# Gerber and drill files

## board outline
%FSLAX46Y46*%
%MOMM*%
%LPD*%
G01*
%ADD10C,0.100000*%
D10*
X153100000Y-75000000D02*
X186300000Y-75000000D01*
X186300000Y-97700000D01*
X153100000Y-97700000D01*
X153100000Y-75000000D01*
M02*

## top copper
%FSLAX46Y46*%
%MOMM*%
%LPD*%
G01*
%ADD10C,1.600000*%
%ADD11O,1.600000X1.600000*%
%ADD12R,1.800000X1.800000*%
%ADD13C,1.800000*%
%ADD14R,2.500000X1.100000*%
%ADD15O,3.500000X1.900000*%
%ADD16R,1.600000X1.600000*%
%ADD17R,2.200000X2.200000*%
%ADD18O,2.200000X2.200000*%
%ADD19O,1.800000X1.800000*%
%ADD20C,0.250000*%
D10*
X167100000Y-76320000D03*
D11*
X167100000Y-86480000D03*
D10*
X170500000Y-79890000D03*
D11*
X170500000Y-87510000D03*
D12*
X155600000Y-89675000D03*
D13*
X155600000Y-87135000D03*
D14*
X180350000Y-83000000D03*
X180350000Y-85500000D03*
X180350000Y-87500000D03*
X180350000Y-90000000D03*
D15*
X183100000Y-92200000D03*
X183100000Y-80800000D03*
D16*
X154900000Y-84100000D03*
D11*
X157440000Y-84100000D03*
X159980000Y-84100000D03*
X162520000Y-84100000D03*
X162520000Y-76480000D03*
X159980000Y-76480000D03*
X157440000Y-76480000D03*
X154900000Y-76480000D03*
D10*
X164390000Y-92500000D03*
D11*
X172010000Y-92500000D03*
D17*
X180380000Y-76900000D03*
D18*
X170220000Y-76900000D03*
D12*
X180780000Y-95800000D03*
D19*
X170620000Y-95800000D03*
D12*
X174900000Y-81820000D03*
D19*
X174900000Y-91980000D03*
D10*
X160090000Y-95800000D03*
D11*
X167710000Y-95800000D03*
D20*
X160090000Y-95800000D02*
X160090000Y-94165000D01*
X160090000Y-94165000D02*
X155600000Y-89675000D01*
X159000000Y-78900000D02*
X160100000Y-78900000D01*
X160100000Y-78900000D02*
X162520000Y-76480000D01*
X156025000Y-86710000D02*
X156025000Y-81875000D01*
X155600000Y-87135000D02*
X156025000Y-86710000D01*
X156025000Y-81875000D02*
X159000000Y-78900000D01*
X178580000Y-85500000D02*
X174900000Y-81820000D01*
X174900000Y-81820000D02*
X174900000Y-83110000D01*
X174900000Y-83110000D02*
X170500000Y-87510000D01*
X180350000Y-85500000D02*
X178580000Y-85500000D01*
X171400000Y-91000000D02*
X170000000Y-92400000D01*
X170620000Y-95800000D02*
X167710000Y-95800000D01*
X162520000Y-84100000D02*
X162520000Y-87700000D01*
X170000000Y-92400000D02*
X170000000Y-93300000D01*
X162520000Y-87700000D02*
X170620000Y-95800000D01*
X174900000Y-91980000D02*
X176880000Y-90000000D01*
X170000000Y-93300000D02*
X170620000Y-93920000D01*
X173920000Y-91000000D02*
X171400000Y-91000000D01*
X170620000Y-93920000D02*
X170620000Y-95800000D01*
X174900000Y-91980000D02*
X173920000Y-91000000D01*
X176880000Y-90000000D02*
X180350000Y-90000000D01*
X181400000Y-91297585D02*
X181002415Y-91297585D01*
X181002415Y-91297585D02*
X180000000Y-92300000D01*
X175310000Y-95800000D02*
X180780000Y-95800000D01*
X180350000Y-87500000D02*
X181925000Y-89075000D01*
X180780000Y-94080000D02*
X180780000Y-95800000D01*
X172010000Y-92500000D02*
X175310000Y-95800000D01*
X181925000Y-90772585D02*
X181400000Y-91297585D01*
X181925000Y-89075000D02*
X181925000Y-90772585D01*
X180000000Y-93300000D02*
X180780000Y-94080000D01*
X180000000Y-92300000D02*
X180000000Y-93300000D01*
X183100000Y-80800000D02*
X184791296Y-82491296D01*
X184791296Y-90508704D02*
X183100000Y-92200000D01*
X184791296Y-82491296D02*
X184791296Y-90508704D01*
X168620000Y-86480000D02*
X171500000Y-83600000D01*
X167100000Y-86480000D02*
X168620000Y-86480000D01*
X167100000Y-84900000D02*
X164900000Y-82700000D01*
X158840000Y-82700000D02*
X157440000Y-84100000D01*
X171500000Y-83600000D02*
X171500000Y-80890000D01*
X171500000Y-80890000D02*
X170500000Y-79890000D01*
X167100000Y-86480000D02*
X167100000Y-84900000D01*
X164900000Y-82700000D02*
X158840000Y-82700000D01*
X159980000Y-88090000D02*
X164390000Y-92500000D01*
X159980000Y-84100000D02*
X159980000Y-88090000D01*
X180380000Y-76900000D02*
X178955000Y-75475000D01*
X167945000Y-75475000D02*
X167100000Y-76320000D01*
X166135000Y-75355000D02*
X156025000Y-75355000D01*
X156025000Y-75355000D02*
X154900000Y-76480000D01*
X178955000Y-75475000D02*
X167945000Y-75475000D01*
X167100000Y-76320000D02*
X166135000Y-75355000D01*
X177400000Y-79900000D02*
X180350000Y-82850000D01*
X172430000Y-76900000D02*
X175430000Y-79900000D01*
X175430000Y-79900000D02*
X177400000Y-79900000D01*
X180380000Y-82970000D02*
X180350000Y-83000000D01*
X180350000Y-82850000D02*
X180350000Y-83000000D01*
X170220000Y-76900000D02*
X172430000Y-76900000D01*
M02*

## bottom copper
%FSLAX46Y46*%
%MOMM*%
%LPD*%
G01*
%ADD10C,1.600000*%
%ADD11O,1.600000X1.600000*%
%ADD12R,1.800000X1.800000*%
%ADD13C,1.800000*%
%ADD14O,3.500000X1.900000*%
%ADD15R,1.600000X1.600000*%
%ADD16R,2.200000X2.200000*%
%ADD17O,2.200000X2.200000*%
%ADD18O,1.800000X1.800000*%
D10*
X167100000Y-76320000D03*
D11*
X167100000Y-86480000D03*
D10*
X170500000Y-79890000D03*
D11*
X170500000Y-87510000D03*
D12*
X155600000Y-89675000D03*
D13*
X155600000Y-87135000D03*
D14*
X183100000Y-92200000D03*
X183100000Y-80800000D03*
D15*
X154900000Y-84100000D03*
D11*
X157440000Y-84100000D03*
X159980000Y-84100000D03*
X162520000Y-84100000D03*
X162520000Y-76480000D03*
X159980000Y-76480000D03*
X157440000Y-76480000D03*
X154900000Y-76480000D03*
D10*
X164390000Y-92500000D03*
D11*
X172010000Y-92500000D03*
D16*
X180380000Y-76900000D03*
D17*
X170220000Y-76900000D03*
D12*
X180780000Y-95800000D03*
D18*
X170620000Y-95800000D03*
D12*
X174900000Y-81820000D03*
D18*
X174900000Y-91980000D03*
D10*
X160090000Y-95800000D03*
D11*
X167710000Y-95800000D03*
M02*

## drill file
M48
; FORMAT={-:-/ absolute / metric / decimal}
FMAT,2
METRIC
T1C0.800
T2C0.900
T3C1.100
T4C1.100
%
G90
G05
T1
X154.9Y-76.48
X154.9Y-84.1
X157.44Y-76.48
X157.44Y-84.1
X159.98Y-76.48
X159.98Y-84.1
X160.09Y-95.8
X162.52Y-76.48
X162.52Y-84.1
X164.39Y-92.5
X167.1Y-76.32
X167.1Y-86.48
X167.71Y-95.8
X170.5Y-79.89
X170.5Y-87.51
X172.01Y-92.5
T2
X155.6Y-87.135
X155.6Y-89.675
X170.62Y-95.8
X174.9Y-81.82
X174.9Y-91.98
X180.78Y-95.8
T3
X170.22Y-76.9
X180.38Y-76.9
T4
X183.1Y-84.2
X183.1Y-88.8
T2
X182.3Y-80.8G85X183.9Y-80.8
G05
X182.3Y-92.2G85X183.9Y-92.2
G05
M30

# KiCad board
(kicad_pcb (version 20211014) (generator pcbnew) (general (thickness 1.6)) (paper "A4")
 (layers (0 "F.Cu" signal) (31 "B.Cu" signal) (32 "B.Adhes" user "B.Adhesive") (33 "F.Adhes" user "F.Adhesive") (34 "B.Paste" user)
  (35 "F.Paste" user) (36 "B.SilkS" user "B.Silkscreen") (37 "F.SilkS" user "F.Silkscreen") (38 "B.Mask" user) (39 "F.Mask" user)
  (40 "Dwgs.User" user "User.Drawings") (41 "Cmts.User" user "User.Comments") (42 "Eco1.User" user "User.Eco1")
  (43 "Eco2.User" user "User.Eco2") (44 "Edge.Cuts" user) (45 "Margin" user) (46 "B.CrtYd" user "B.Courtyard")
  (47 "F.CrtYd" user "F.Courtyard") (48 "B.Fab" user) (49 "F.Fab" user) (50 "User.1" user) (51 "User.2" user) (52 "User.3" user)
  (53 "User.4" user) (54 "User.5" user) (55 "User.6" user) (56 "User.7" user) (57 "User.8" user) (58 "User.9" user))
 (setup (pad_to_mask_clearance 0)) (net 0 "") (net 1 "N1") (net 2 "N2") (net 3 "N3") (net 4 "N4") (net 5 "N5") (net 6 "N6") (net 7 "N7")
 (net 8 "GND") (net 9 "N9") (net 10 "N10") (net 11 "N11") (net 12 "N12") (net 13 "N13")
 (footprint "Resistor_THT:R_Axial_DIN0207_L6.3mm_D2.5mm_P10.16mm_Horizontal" (layer "F.Cu") (at 167.1 76.32 -90)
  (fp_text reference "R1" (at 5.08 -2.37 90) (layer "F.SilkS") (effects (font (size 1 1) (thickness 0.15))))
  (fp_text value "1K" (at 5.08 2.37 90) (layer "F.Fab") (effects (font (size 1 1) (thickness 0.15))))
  (pad "1" thru_hole circle (at 0 0 270) (size 1.6 1.6) (drill 0.8) (layers *.Cu *.Mask) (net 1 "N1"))
  (pad "2" thru_hole oval (at 10.16 0 270) (size 1.6 1.6) (drill 0.8) (layers *.Cu *.Mask) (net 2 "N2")))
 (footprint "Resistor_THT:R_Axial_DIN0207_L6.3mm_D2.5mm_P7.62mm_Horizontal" (layer "F.Cu") (at 170.5 79.89 -90)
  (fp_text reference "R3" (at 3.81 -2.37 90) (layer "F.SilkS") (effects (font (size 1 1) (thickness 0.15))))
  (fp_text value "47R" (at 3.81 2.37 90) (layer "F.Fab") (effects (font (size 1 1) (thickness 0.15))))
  (pad "1" thru_hole circle (at 0 0 270) (size 1.6 1.6) (drill 0.8) (layers *.Cu *.Mask) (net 2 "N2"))
  (pad "2" thru_hole oval (at 7.62 0 270) (size 1.6 1.6) (drill 0.8) (layers *.Cu *.Mask) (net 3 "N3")))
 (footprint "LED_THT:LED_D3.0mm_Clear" (layer "F.Cu") (at 155.6 89.675 90)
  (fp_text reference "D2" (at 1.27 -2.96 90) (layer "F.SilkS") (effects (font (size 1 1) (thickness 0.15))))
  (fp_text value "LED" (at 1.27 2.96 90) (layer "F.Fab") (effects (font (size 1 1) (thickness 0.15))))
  (pad "1" thru_hole rect (at 0 0 90) (size 1.8 1.8) (drill 0.9) (layers *.Cu *.Mask) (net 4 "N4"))
  (pad "2" thru_hole circle (at 2.54 0 90) (size 1.8 1.8) (drill 0.9) (layers *.Cu *.Mask) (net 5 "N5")))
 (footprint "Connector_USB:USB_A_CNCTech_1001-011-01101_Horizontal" (layer "F.Cu") (at 190 86.5)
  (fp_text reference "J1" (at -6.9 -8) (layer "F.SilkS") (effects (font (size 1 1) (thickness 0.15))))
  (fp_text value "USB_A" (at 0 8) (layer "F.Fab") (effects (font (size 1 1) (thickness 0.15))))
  (pad "" np_thru_hole circle (at -6.9 -2.3) (size 1.1 1.1) (drill 1.1) (layers *.Cu *.Mask))
  (pad "" np_thru_hole circle (at -6.9 2.3) (size 1.1 1.1) (drill 1.1) (layers *.Cu *.Mask))
  (pad "1" smd rect (at -9.65 -3.5) (size 2.5 1.1) (layers "F.Cu" "F.Paste" "F.Mask") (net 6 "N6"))
  (pad "2" smd rect (at -9.65 -1) (size 2.5 1.1) (layers "F.Cu" "F.Paste" "F.Mask") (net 3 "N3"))
  (pad "3" smd rect (at -9.65 1) (size 2.5 1.1) (layers "F.Cu" "F.Paste" "F.Mask") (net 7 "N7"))
  (pad "4" smd rect (at -9.65 3.5) (size 2.5 1.1) (layers "F.Cu" "F.Paste" "F.Mask") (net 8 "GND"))
  (pad "5" thru_hole oval (at -6.9 5.7) (size 3.5 1.9) (drill oval 2.5 0.9) (layers *.Cu *.Mask) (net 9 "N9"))
  (pad "5" thru_hole oval (at -6.9 -5.7) (size 3.5 1.9) (drill oval 2.5 0.9) (layers *.Cu *.Mask) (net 9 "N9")))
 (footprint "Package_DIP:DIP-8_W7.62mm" (layer "F.Cu") (at 154.9 84.1 90)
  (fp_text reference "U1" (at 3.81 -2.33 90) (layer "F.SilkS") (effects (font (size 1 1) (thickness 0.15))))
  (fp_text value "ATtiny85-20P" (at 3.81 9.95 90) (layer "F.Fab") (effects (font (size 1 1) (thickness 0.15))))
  (pad "1" thru_hole rect (at 0 0 90) (size 1.6 1.6) (drill 0.8) (layers *.Cu *.Mask) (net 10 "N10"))
  (pad "2" thru_hole oval (at 0 2.54 90) (size 1.6 1.6) (drill 0.8) (layers *.Cu *.Mask) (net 2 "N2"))
  (pad "3" thru_hole oval (at 0 5.08 90) (size 1.6 1.6) (drill 0.8) (layers *.Cu *.Mask) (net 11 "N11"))
  (pad "4" thru_hole oval (at 0 7.62 90) (size 1.6 1.6) (drill 0.8) (layers *.Cu *.Mask) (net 8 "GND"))
  (pad "5" thru_hole oval (at 7.62 7.62 90) (size 1.6 1.6) (drill 0.8) (layers *.Cu *.Mask) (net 5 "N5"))
  (pad "6" thru_hole oval (at 7.62 5.08 90) (size 1.6 1.6) (drill 0.8) (layers *.Cu *.Mask) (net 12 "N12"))
  (pad "7" thru_hole oval (at 7.62 2.54 90) (size 1.6 1.6) (drill 0.8) (layers *.Cu *.Mask) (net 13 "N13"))
  (pad "8" thru_hole oval (at 7.62 0 90) (size 1.6 1.6) (drill 0.8) (layers *.Cu *.Mask) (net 1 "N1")))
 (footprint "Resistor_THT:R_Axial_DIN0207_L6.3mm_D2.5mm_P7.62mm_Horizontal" (layer "F.Cu") (at 164.39 92.5)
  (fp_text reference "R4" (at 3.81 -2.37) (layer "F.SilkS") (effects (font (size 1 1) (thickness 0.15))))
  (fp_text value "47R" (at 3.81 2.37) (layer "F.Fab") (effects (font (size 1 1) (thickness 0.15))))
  (pad "1" thru_hole circle (at 0 0) (size 1.6 1.6) (drill 0.8) (layers *.Cu *.Mask) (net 11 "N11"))
  (pad "2" thru_hole oval (at 7.62 0) (size 1.6 1.6) (drill 0.8) (layers *.Cu *.Mask) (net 7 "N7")))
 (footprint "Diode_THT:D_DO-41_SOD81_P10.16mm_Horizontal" (layer "F.Cu") (at 180.38 76.9 180)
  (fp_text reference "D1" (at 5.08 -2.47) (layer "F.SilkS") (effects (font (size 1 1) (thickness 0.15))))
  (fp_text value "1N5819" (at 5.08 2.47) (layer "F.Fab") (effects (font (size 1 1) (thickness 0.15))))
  (pad "1" thru_hole rect (at 0 0 180) (size 2.2 2.2) (drill 1.1) (layers *.Cu *.Mask) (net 1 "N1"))
  (pad "2" thru_hole oval (at 10.16 0 180) (size 2.2 2.2) (drill 1.1) (layers *.Cu *.Mask) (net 6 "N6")))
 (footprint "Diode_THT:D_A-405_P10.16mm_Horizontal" (layer "F.Cu") (at 180.78 95.8 180)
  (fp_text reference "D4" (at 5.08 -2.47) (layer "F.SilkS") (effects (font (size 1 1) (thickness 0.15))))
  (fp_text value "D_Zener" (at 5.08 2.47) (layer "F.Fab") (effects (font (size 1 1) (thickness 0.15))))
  (pad "1" thru_hole rect (at 0 0 180) (size 1.8 1.8) (drill 0.9) (layers *.Cu *.Mask) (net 7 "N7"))
  (pad "2" thru_hole oval (at 10.16 0 180) (size 1.8 1.8) (drill 0.9) (layers *.Cu *.Mask) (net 8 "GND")))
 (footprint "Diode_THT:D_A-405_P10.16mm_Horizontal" (layer "F.Cu") (at 174.9 81.82 -90)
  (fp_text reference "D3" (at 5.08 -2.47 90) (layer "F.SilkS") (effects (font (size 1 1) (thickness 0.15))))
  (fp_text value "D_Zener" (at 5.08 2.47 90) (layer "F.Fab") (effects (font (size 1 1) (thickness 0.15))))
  (pad "1" thru_hole rect (at 0 0 270) (size 1.8 1.8) (drill 0.9) (layers *.Cu *.Mask) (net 3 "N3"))
  (pad "2" thru_hole oval (at 10.16 0 270) (size 1.8 1.8) (drill 0.9) (layers *.Cu *.Mask) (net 8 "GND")))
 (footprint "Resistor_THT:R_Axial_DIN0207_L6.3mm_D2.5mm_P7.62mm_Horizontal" (layer "F.Cu") (at 160.09 95.8)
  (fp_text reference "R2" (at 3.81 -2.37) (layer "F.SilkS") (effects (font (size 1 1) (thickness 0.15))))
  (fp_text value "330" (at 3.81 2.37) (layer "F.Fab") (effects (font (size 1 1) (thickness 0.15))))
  (pad "1" thru_hole circle (at 0 0) (size 1.6 1.6) (drill 0.8) (layers *.Cu *.Mask) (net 4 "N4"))
  (pad "2" thru_hole oval (at 7.62 0) (size 1.6 1.6) (drill 0.8) (layers *.Cu *.Mask) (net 8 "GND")))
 (gr_rect (start 186.3 75) (end 153.1 97.7) (layer "Edge.Cuts") (width 0.1) (fill none))
 (segment (start 160.09 95.8) (end 160.09 94.165) (width 0.25) (layer "F.Cu") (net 4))
 (segment (start 160.09 94.165) (end 155.6 89.675) (width 0.25) (layer "F.Cu") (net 4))
 (segment (start 159 78.9) (end 160.1 78.9) (width 0.25) (layer "F.Cu") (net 5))
 (segment (start 160.1 78.9) (end 162.52 76.48) (width 0.25) (layer "F.Cu") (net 5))
 (segment (start 156.025 86.71) (end 156.025 81.875) (width 0.25) (layer "F.Cu") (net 5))
 (segment (start 155.6 87.135) (end 156.025 86.71) (width 0.25) (layer "F.Cu") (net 5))
 (segment (start 156.025 81.875) (end 159 78.9) (width 0.25) (layer "F.Cu") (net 5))
 (segment (start 178.58 85.5) (end 174.9 81.82) (width 0.25) (layer "F.Cu") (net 3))
 (segment (start 174.9 81.82) (end 174.9 83.11) (width 0.25) (layer "F.Cu") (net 3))
 (segment (start 174.9 83.11) (end 170.5 87.51) (width 0.25) (layer "F.Cu") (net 3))
 (segment (start 180.35 85.5) (end 178.58 85.5) (width 0.25) (layer "F.Cu") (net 3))
 (segment (start 171.4 91) (end 170 92.4) (width 0.25) (layer "F.Cu") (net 8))
 (segment (start 170.62 95.8) (end 167.71 95.8) (width 0.25) (layer "F.Cu") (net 8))
 (segment (start 162.52 84.1) (end 162.52 87.7) (width 0.25) (layer "F.Cu") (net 8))
 (segment (start 170 92.4) (end 170 93.3) (width 0.25) (layer "F.Cu") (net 8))
 (segment (start 162.52 87.7) (end 170.62 95.8) (width 0.25) (layer "F.Cu") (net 8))
 (segment (start 174.9 91.98) (end 176.88 90) (width 0.25) (layer "F.Cu") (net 8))
 (segment (start 170 93.3) (end 170.62 93.92) (width 0.25) (layer "F.Cu") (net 8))
 (segment (start 173.92 91) (end 171.4 91) (width 0.25) (layer "F.Cu") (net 8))
 (segment (start 170.62 93.92) (end 170.62 95.8) (width 0.25) (layer "F.Cu") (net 8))
 (segment (start 174.9 91.98) (end 173.92 91) (width 0.25) (layer "F.Cu") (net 8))
 (segment (start 176.88 90) (end 180.35 90) (width 0.25) (layer "F.Cu") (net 8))
 (segment (start 181.4 91.297585) (end 181.002415 91.297585) (width 0.25) (layer "F.Cu") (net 7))
 (segment (start 181.002415 91.297585) (end 180 92.3) (width 0.25) (layer "F.Cu") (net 7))
 (segment (start 175.31 95.8) (end 180.78 95.8) (width 0.25) (layer "F.Cu") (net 7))
 (segment (start 180.35 87.5) (end 181.925 89.075) (width 0.25) (layer "F.Cu") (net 7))
 (segment (start 180.78 94.08) (end 180.78 95.8) (width 0.25) (layer "F.Cu") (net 7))
 (segment (start 172.01 92.5) (end 175.31 95.8) (width 0.25) (layer "F.Cu") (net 7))
 (segment (start 181.925 90.772585) (end 181.4 91.297585) (width 0.25) (layer "F.Cu") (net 7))
 (segment (start 181.925 89.075) (end 181.925 90.772585) (width 0.25) (layer "F.Cu") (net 7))
 (segment (start 180 93.3) (end 180.78 94.08) (width 0.25) (layer "F.Cu") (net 7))
 (segment (start 180 92.3) (end 180 93.3) (width 0.25) (layer "F.Cu") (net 7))
 (segment (start 183.1 80.8) (end 184.791296 82.491296) (width 0.25) (layer "F.Cu") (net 9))
 (segment (start 184.791296 90.508704) (end 183.1 92.2) (width 0.25) (layer "F.Cu") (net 9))
 (segment (start 184.791296 82.491296) (end 184.791296 90.508704) (width 0.25) (layer "F.Cu") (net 9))
 (segment (start 168.62 86.48) (end 171.5 83.6) (width 0.25) (layer "F.Cu") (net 2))
 (segment (start 167.1 86.48) (end 168.62 86.48) (width 0.25) (layer "F.Cu") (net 2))
 (segment (start 167.1 84.9) (end 164.9 82.7) (width 0.25) (layer "F.Cu") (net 2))
 (segment (start 158.84 82.7) (end 157.44 84.1) (width 0.25) (layer "F.Cu") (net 2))
 (segment (start 171.5 83.6) (end 171.5 80.89) (width 0.25) (layer "F.Cu") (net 2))
 (segment (start 171.5 80.89) (end 170.5 79.89) (width 0.25) (layer "F.Cu") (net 2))
 (segment (start 167.1 86.48) (end 167.1 84.9) (width 0.25) (layer "F.Cu") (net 2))
 (segment (start 164.9 82.7) (end 158.84 82.7) (width 0.25) (layer "F.Cu") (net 2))
 (segment (start 159.98 88.09) (end 164.39 92.5) (width 0.25) (layer "F.Cu") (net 11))
 (segment (start 159.98 84.1) (end 159.98 88.09) (width 0.25) (layer "F.Cu") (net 11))
 (segment (start 180.38 76.9) (end 178.955 75.475) (width 0.25) (layer "F.Cu") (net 1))
 (segment (start 167.945 75.475) (end 167.1 76.32) (width 0.25) (layer "F.Cu") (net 1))
 (segment (start 166.135 75.355) (end 156.025 75.355) (width 0.25) (layer "F.Cu") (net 1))
 (segment (start 156.025 75.355) (end 154.9 76.48) (width 0.25) (layer "F.Cu") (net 1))
 (segment (start 178.955 75.475) (end 167.945 75.475) (width 0.25) (layer "F.Cu") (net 1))
 (segment (start 167.1 76.32) (end 166.135 75.355) (width 0.25) (layer "F.Cu") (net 1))
 (segment (start 177.4 79.9) (end 180.35 82.85) (width 0.25) (layer "F.Cu") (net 6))
 (segment (start 172.43 76.9) (end 175.43 79.9) (width 0.25) (layer "F.Cu") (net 6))
 (segment (start 175.43 79.9) (end 177.4 79.9) (width 0.25) (layer "F.Cu") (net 6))
 (segment (start 180.38 82.97) (end 180.35 83) (width 0.25) (layer "F.Cu") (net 6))
 (segment (start 180.35 82.85) (end 180.35 83) (width 0.25) (layer "F.Cu") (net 6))
 (segment (start 170.22 76.9) (end 172.43 76.9) (width 0.25) (layer "F.Cu") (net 6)))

